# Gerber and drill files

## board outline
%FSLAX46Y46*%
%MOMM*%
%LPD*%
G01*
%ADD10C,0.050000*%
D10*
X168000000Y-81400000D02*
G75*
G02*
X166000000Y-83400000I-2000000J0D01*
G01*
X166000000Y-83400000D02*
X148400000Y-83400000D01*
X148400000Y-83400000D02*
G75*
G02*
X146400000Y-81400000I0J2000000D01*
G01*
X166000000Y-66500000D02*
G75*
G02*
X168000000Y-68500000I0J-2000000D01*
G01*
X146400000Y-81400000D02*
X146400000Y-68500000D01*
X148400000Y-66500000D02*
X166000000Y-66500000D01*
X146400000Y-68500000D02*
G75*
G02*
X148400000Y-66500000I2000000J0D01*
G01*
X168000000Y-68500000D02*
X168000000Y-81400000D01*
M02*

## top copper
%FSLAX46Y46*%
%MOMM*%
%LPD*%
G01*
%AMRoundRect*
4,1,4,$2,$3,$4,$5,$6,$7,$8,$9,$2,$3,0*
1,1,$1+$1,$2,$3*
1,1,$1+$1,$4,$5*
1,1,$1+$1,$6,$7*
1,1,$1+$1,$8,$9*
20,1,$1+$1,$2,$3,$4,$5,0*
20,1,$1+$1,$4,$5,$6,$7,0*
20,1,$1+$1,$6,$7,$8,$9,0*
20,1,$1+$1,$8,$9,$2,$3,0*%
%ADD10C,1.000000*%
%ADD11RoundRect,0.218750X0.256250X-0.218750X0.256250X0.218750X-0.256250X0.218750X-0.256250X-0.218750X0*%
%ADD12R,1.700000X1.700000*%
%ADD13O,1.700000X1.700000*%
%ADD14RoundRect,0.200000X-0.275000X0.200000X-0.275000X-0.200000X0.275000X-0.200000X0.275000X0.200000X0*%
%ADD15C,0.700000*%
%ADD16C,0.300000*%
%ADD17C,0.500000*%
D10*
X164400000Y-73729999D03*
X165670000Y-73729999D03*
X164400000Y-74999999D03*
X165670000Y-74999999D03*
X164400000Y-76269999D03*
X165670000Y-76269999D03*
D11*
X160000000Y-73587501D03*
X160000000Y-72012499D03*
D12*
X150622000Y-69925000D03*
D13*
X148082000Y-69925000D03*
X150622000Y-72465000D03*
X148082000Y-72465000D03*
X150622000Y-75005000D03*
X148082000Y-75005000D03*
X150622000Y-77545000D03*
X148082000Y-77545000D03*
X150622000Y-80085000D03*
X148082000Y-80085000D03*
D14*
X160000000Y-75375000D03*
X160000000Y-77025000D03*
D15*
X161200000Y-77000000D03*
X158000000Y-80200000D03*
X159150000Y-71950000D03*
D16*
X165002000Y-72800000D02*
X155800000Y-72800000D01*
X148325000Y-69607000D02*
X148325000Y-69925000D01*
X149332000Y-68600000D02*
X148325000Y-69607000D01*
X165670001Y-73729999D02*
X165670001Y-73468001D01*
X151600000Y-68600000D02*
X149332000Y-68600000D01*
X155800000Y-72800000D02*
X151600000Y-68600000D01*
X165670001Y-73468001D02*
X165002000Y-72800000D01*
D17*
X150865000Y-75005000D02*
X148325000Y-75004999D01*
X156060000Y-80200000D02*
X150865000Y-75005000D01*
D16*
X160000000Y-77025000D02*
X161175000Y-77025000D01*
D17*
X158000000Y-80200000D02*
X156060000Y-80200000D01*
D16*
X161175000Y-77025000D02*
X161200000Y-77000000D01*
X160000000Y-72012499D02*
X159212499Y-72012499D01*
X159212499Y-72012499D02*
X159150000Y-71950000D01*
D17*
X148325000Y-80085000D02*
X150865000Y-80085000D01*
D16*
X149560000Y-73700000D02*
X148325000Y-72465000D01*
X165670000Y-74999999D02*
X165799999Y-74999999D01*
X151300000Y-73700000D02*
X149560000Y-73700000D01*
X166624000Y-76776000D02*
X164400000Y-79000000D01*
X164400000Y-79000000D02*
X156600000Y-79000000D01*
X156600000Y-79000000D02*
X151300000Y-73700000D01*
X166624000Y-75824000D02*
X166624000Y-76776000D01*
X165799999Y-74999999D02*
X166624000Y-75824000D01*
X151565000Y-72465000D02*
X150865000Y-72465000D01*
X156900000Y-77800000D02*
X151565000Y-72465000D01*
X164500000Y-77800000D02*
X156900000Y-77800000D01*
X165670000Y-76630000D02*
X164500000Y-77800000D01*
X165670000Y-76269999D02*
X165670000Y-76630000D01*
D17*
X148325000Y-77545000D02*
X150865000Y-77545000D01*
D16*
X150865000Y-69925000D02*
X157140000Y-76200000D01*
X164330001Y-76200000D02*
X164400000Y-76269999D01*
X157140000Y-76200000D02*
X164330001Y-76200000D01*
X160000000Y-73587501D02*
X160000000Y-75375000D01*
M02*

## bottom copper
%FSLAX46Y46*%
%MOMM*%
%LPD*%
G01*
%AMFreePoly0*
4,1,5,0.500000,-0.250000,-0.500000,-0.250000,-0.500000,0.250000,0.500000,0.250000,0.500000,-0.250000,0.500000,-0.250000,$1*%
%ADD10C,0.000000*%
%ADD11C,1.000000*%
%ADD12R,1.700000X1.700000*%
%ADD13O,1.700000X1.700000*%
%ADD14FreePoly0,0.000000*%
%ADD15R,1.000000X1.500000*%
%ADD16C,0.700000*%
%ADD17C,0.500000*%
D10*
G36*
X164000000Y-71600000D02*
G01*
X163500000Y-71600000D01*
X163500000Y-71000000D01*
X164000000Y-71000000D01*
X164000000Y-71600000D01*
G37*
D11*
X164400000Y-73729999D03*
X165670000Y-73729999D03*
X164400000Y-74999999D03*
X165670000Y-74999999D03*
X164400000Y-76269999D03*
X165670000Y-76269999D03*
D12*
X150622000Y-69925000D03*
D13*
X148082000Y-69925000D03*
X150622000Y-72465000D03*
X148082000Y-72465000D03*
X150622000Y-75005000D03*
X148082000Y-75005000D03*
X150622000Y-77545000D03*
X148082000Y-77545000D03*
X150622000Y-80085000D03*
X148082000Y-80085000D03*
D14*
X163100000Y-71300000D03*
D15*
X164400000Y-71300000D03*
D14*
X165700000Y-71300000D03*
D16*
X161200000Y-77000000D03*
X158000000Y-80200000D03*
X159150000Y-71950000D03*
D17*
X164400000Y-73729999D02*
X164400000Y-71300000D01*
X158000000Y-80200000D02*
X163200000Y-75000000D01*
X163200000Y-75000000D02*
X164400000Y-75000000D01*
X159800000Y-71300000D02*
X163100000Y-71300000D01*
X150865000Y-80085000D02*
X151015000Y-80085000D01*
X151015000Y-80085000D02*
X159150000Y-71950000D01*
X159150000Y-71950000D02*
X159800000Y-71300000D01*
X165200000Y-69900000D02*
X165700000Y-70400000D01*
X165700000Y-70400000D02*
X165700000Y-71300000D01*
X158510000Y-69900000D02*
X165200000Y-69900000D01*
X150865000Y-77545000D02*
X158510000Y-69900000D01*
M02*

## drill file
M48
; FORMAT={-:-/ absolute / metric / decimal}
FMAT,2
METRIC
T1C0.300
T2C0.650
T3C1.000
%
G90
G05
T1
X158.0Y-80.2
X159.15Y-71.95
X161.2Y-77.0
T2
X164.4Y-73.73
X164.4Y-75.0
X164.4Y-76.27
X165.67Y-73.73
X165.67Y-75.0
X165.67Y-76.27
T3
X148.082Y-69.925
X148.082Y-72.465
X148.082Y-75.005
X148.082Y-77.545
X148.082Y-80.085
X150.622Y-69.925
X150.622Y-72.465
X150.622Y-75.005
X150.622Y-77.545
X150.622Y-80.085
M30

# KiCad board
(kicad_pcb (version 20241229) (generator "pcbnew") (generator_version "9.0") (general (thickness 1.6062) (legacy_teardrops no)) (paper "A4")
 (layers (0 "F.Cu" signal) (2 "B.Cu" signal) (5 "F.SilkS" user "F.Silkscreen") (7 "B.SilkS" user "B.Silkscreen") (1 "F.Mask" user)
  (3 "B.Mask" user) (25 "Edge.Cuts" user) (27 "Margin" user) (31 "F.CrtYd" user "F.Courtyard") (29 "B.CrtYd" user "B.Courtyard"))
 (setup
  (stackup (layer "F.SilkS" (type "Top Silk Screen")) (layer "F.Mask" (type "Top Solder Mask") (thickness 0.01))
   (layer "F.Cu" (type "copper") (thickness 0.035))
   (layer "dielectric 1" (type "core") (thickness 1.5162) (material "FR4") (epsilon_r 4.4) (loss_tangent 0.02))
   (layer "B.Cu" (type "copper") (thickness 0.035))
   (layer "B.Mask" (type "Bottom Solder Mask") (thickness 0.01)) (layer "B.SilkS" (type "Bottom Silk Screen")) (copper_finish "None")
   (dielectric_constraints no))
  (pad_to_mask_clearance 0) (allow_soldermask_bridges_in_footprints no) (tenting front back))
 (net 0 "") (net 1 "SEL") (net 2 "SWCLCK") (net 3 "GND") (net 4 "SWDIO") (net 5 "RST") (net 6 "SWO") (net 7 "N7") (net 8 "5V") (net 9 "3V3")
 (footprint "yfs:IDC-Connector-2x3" (layer "F.Cu") (at 164.4 73.729999 -90)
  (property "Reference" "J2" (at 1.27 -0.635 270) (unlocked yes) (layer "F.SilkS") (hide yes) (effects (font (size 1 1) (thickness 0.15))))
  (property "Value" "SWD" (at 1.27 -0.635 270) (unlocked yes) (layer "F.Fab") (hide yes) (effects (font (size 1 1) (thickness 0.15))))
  (pad "1" thru_hole circle (at 0 0 270) (size 1 1) (drill 0.65) (layers "*.Cu" "*.Mask") (remove_unused_layers no) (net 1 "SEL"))
  (pad "2" thru_hole circle (at 0 -1.27 270) (size 1 1) (drill 0.65) (layers "*.Cu" "*.Mask") (remove_unused_layers no) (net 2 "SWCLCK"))
  (pad "3" thru_hole circle (at 1.27 0 270) (size 1 1) (drill 0.65) (layers "*.Cu" "*.Mask") (remove_unused_layers no) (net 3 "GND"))
  (pad "4" thru_hole circle (at 1.27 -1.27 270) (size 1 1) (drill 0.65) (layers "*.Cu" "*.Mask") (remove_unused_layers no) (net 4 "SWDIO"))
  (pad "5" thru_hole circle (at 2.54 0 270) (size 1 1) (drill 0.65) (layers "*.Cu" "*.Mask") (remove_unused_layers no) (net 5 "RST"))
  (pad "6" thru_hole circle (at 2.54 -1.27 270) (size 1 1) (drill 0.65) (layers "*.Cu" "*.Mask") (remove_unused_layers no) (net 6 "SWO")))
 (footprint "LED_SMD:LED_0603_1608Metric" (layer "F.Cu") (at 160 72.8 90)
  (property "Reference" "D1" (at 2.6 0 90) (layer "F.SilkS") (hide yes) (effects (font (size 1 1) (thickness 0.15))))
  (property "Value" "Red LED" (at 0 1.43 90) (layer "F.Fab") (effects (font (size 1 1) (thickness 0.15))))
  (pad "1" smd roundrect (at -0.787501 0 90) (size 0.875 0.95) (layers "F.Cu" "F.Mask" "F.Paste") (roundrect_rratio 0.25) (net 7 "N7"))
  (pad "2" smd roundrect (at 0.787501 0 90) (size 0.875 0.95) (layers "F.Cu" "F.Mask" "F.Paste") (roundrect_rratio 0.25) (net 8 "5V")))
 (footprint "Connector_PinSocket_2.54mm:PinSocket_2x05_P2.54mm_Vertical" (layer "F.Cu") (at 150.622 69.925)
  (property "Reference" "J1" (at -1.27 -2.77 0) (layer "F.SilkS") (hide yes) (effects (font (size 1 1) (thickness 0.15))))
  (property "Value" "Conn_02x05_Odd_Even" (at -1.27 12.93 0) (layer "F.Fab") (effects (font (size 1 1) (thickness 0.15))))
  (pad "1" thru_hole rect (at 0 0) (size 1.7 1.7) (drill 1) (layers "*.Cu" "*.Mask") (remove_unused_layers no) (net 5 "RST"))
  (pad "2" thru_hole oval (at -2.54 0) (size 1.7 1.7) (drill 1) (layers "*.Cu" "*.Mask") (remove_unused_layers no) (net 2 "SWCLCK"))
  (pad "3" thru_hole oval (at 0 2.54) (size 1.7 1.7) (drill 1) (layers "*.Cu" "*.Mask") (remove_unused_layers no) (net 6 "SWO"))
  (pad "4" thru_hole oval (at -2.54 2.54) (size 1.7 1.7) (drill 1) (layers "*.Cu" "*.Mask") (remove_unused_layers no) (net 4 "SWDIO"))
  (pad "5" thru_hole oval (at 0 5.08) (size 1.7 1.7) (drill 1) (layers "*.Cu" "*.Mask") (remove_unused_layers no) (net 3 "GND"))
  (pad "6" thru_hole oval (at -2.54 5.08) (size 1.7 1.7) (drill 1) (layers "*.Cu" "*.Mask") (remove_unused_layers no) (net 3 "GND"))
  (pad "7" thru_hole oval (at 0 7.62) (size 1.7 1.7) (drill 1) (layers "*.Cu" "*.Mask") (remove_unused_layers no) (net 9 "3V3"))
  (pad "8" thru_hole oval (at -2.54 7.62) (size 1.7 1.7) (drill 1) (layers "*.Cu" "*.Mask") (remove_unused_layers no) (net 9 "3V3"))
  (pad "9" thru_hole oval (at 0 10.16) (size 1.7 1.7) (drill 1) (layers "*.Cu" "*.Mask") (remove_unused_layers no) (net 8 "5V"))
  (pad "10" thru_hole oval (at -2.54 10.16) (size 1.7 1.7) (drill 1) (layers "*.Cu" "*.Mask") (remove_unused_layers no) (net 8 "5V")))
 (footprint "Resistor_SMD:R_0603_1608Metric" (layer "F.Cu") (at 160 76.2 -90)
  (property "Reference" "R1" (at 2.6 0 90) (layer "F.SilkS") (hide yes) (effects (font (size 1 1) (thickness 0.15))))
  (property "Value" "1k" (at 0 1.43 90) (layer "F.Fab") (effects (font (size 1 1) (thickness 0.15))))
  (pad "1" smd roundrect (at -0.825 0 270) (size 0.8 0.95) (layers "F.Cu" "F.Mask" "F.Paste") (roundrect_rratio 0.25) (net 7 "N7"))
  (pad "2" smd roundrect (at 0.825 0 270) (size 0.8 0.95) (layers "F.Cu" "F.Mask" "F.Paste") (roundrect_rratio 0.25) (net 3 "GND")))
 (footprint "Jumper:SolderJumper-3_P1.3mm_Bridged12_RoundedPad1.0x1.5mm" (layer "B.Cu") (at 164.4 71.3)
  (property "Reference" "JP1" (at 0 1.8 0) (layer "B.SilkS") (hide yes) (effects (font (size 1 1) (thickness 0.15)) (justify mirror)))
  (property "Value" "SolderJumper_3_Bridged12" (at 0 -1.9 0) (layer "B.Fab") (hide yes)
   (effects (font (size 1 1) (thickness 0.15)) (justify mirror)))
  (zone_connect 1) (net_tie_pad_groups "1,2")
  (fp_poly (pts (xy -0.9 0.3) (xy -0.4 0.3) (xy -0.4 -0.3) (xy -0.9 -0.3)) (stroke (width 0) (type solid)) (fill yes) (layer "B.Cu"))
  (pad "1" smd custom (at -1.3 0) (size 1 0.5) (layers "B.Cu" "B.Mask") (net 8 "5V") (zone_connect 2) (thermal_bridge_angle 45)
   (options (clearance outline) (anchor rect)) (primitives))
  (pad "2" smd rect (at 0 0) (size 1 1.5) (layers "B.Cu" "B.Mask") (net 1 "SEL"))
  (pad "3" smd custom (at 1.3 0) (size 1 0.5) (layers "B.Cu" "B.Mask") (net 9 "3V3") (zone_connect 2) (thermal_bridge_angle 45)
   (options (clearance outline) (anchor rect)) (primitives)))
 (gr_arc (start 168 81.4) (mid 167.414214 82.814214) (end 166 83.4) (stroke (width 0.05) (type default)) (layer "Edge.Cuts"))
 (gr_line (start 166 83.4) (end 148.4 83.4) (stroke (width 0.05) (type default)) (layer "Edge.Cuts"))
 (gr_arc (start 148.4 83.4) (mid 146.985786 82.814214) (end 146.4 81.4) (stroke (width 0.05) (type default)) (layer "Edge.Cuts"))
 (gr_arc (start 166 66.5) (mid 167.414214 67.085786) (end 168 68.5) (stroke (width 0.05) (type default)) (layer "Edge.Cuts"))
 (gr_line (start 146.4 81.4) (end 146.4 68.5) (stroke (width 0.05) (type default)) (layer "Edge.Cuts"))
 (gr_line (start 148.4 66.5) (end 166 66.5) (stroke (width 0.05) (type default)) (layer "Edge.Cuts"))
 (gr_arc (start 146.4 68.5) (mid 146.985786 67.085786) (end 148.4 66.5) (stroke (width 0.05) (type default)) (layer "Edge.Cuts"))
 (gr_line (start 168 68.5) (end 168 81.4) (stroke (width 0.05) (type default)) (layer "Edge.Cuts"))
 (segment (start 164.4 73.729999) (end 164.4 71.3) (width 0.5) (layer "B.Cu") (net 1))
 (segment (start 165.002 72.8) (end 155.8 72.8) (width 0.3) (layer "F.Cu") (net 2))
 (segment (start 148.325 69.607) (end 148.325 69.925) (width 0.3) (layer "F.Cu") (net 2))
 (segment (start 149.332 68.6) (end 148.325 69.607) (width 0.3) (layer "F.Cu") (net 2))
 (segment (start 165.670001 73.729999) (end 165.670001 73.468001) (width 0.3) (layer "F.Cu") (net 2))
 (segment (start 151.6 68.6) (end 149.332 68.6) (width 0.3) (layer "F.Cu") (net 2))
 (segment (start 155.8 72.8) (end 151.6 68.6) (width 0.3) (layer "F.Cu") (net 2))
 (segment (start 165.670001 73.468001) (end 165.002 72.8) (width 0.3) (layer "F.Cu") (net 2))
 (segment (start 150.865 75.005) (end 148.325 75.004999) (width 0.5) (layer "F.Cu") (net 3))
 (segment (start 156.06 80.2) (end 150.865 75.005) (width 0.5) (layer "F.Cu") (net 3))
 (segment (start 160 77.025) (end 161.175 77.025) (width 0.3) (layer "F.Cu") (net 3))
 (segment (start 158 80.2) (end 156.06 80.2) (width 0.5) (layer "F.Cu") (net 3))
 (segment (start 161.175 77.025) (end 161.2 77) (width 0.3) (layer "F.Cu") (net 3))
 (via (at 161.2 77) (size 0.7) (drill 0.3) (layers "F.Cu" "B.Cu") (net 3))
 (via (at 158 80.2) (size 0.7) (drill 0.3) (layers "F.Cu" "B.Cu") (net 3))
 (segment (start 158 80.2) (end 163.2 75) (width 0.5) (layer "B.Cu") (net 3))
 (segment (start 163.2 75) (end 164.4 75) (width 0.5) (layer "B.Cu") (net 3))
 (segment (start 160 72.012499) (end 159.212499 72.012499) (width 0.3) (layer "F.Cu") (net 8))
 (segment (start 159.212499 72.012499) (end 159.15 71.95) (width 0.3) (layer "F.Cu") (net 8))
 (segment (start 148.325 80.085) (end 150.865 80.085) (width 0.5) (layer "F.Cu") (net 8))
 (via (at 159.15 71.95) (size 0.7) (drill 0.3) (layers "F.Cu" "B.Cu") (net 8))
 (segment (start 159.8 71.3) (end 163.1 71.3) (width 0.5) (layer "B.Cu") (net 8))
 (segment (start 150.865 80.085) (end 151.015 80.085) (width 0.5) (layer "B.Cu") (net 8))
 (segment (start 151.015 80.085) (end 159.15 71.95) (width 0.5) (layer "B.Cu") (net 8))
 (segment (start 159.15 71.95) (end 159.8 71.3) (width 0.5) (layer "B.Cu") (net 8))
 (segment (start 149.56 73.7) (end 148.325 72.465) (width 0.3) (layer "F.Cu") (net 4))
 (segment (start 165.67 74.999999) (end 165.799999 74.999999) (width 0.3) (layer "F.Cu") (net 4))
 (segment (start 151.3 73.7) (end 149.56 73.7) (width 0.3) (layer "F.Cu") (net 4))
 (segment (start 166.624 76.776) (end 164.4 79) (width 0.3) (layer "F.Cu") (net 4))
 (segment (start 164.4 79) (end 156.6 79) (width 0.3) (layer "F.Cu") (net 4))
 (segment (start 156.6 79) (end 151.3 73.7) (width 0.3) (layer "F.Cu") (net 4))
 (segment (start 166.624 75.824) (end 166.624 76.776) (width 0.3) (layer "F.Cu") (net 4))
 (segment (start 165.799999 74.999999) (end 166.624 75.824) (width 0.3) (layer "F.Cu") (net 4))
 (segment (start 151.565 72.465) (end 150.865 72.465) (width 0.3) (layer "F.Cu") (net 6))
 (segment (start 156.9 77.8) (end 151.565 72.465) (width 0.3) (layer "F.Cu") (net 6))
 (segment (start 164.5 77.8) (end 156.9 77.8) (width 0.3) (layer "F.Cu") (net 6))
 (segment (start 165.67 76.63) (end 164.5 77.8) (width 0.3) (layer "F.Cu") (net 6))
 (segment (start 165.67 76.269999) (end 165.67 76.63) (width 0.3) (layer "F.Cu") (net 6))
 (segment (start 148.325 77.545) (end 150.865 77.545) (width 0.5) (layer "F.Cu") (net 9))
 (segment (start 165.2 69.9) (end 165.7 70.4) (width 0.5) (layer "B.Cu") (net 9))
 (segment (start 165.7 70.4) (end 165.7 71.3) (width 0.5) (layer "B.Cu") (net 9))
 (segment (start 158.51 69.9) (end 165.2 69.9) (width 0.5) (layer "B.Cu") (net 9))
 (segment (start 150.865 77.545) (end 158.51 69.9) (width 0.5) (layer "B.Cu") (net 9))
 (segment (start 150.865 69.925) (end 157.14 76.2) (width 0.3) (layer "F.Cu") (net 5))
 (segment (start 164.330001 76.2) (end 164.4 76.269999) (width 0.3) (layer "F.Cu") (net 5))
 (segment (start 157.14 76.2) (end 164.330001 76.2) (width 0.3) (layer "F.Cu") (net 5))
 (segment (start 160 73.587501) (end 160 75.375) (width 0.3) (layer "F.Cu") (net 7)))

